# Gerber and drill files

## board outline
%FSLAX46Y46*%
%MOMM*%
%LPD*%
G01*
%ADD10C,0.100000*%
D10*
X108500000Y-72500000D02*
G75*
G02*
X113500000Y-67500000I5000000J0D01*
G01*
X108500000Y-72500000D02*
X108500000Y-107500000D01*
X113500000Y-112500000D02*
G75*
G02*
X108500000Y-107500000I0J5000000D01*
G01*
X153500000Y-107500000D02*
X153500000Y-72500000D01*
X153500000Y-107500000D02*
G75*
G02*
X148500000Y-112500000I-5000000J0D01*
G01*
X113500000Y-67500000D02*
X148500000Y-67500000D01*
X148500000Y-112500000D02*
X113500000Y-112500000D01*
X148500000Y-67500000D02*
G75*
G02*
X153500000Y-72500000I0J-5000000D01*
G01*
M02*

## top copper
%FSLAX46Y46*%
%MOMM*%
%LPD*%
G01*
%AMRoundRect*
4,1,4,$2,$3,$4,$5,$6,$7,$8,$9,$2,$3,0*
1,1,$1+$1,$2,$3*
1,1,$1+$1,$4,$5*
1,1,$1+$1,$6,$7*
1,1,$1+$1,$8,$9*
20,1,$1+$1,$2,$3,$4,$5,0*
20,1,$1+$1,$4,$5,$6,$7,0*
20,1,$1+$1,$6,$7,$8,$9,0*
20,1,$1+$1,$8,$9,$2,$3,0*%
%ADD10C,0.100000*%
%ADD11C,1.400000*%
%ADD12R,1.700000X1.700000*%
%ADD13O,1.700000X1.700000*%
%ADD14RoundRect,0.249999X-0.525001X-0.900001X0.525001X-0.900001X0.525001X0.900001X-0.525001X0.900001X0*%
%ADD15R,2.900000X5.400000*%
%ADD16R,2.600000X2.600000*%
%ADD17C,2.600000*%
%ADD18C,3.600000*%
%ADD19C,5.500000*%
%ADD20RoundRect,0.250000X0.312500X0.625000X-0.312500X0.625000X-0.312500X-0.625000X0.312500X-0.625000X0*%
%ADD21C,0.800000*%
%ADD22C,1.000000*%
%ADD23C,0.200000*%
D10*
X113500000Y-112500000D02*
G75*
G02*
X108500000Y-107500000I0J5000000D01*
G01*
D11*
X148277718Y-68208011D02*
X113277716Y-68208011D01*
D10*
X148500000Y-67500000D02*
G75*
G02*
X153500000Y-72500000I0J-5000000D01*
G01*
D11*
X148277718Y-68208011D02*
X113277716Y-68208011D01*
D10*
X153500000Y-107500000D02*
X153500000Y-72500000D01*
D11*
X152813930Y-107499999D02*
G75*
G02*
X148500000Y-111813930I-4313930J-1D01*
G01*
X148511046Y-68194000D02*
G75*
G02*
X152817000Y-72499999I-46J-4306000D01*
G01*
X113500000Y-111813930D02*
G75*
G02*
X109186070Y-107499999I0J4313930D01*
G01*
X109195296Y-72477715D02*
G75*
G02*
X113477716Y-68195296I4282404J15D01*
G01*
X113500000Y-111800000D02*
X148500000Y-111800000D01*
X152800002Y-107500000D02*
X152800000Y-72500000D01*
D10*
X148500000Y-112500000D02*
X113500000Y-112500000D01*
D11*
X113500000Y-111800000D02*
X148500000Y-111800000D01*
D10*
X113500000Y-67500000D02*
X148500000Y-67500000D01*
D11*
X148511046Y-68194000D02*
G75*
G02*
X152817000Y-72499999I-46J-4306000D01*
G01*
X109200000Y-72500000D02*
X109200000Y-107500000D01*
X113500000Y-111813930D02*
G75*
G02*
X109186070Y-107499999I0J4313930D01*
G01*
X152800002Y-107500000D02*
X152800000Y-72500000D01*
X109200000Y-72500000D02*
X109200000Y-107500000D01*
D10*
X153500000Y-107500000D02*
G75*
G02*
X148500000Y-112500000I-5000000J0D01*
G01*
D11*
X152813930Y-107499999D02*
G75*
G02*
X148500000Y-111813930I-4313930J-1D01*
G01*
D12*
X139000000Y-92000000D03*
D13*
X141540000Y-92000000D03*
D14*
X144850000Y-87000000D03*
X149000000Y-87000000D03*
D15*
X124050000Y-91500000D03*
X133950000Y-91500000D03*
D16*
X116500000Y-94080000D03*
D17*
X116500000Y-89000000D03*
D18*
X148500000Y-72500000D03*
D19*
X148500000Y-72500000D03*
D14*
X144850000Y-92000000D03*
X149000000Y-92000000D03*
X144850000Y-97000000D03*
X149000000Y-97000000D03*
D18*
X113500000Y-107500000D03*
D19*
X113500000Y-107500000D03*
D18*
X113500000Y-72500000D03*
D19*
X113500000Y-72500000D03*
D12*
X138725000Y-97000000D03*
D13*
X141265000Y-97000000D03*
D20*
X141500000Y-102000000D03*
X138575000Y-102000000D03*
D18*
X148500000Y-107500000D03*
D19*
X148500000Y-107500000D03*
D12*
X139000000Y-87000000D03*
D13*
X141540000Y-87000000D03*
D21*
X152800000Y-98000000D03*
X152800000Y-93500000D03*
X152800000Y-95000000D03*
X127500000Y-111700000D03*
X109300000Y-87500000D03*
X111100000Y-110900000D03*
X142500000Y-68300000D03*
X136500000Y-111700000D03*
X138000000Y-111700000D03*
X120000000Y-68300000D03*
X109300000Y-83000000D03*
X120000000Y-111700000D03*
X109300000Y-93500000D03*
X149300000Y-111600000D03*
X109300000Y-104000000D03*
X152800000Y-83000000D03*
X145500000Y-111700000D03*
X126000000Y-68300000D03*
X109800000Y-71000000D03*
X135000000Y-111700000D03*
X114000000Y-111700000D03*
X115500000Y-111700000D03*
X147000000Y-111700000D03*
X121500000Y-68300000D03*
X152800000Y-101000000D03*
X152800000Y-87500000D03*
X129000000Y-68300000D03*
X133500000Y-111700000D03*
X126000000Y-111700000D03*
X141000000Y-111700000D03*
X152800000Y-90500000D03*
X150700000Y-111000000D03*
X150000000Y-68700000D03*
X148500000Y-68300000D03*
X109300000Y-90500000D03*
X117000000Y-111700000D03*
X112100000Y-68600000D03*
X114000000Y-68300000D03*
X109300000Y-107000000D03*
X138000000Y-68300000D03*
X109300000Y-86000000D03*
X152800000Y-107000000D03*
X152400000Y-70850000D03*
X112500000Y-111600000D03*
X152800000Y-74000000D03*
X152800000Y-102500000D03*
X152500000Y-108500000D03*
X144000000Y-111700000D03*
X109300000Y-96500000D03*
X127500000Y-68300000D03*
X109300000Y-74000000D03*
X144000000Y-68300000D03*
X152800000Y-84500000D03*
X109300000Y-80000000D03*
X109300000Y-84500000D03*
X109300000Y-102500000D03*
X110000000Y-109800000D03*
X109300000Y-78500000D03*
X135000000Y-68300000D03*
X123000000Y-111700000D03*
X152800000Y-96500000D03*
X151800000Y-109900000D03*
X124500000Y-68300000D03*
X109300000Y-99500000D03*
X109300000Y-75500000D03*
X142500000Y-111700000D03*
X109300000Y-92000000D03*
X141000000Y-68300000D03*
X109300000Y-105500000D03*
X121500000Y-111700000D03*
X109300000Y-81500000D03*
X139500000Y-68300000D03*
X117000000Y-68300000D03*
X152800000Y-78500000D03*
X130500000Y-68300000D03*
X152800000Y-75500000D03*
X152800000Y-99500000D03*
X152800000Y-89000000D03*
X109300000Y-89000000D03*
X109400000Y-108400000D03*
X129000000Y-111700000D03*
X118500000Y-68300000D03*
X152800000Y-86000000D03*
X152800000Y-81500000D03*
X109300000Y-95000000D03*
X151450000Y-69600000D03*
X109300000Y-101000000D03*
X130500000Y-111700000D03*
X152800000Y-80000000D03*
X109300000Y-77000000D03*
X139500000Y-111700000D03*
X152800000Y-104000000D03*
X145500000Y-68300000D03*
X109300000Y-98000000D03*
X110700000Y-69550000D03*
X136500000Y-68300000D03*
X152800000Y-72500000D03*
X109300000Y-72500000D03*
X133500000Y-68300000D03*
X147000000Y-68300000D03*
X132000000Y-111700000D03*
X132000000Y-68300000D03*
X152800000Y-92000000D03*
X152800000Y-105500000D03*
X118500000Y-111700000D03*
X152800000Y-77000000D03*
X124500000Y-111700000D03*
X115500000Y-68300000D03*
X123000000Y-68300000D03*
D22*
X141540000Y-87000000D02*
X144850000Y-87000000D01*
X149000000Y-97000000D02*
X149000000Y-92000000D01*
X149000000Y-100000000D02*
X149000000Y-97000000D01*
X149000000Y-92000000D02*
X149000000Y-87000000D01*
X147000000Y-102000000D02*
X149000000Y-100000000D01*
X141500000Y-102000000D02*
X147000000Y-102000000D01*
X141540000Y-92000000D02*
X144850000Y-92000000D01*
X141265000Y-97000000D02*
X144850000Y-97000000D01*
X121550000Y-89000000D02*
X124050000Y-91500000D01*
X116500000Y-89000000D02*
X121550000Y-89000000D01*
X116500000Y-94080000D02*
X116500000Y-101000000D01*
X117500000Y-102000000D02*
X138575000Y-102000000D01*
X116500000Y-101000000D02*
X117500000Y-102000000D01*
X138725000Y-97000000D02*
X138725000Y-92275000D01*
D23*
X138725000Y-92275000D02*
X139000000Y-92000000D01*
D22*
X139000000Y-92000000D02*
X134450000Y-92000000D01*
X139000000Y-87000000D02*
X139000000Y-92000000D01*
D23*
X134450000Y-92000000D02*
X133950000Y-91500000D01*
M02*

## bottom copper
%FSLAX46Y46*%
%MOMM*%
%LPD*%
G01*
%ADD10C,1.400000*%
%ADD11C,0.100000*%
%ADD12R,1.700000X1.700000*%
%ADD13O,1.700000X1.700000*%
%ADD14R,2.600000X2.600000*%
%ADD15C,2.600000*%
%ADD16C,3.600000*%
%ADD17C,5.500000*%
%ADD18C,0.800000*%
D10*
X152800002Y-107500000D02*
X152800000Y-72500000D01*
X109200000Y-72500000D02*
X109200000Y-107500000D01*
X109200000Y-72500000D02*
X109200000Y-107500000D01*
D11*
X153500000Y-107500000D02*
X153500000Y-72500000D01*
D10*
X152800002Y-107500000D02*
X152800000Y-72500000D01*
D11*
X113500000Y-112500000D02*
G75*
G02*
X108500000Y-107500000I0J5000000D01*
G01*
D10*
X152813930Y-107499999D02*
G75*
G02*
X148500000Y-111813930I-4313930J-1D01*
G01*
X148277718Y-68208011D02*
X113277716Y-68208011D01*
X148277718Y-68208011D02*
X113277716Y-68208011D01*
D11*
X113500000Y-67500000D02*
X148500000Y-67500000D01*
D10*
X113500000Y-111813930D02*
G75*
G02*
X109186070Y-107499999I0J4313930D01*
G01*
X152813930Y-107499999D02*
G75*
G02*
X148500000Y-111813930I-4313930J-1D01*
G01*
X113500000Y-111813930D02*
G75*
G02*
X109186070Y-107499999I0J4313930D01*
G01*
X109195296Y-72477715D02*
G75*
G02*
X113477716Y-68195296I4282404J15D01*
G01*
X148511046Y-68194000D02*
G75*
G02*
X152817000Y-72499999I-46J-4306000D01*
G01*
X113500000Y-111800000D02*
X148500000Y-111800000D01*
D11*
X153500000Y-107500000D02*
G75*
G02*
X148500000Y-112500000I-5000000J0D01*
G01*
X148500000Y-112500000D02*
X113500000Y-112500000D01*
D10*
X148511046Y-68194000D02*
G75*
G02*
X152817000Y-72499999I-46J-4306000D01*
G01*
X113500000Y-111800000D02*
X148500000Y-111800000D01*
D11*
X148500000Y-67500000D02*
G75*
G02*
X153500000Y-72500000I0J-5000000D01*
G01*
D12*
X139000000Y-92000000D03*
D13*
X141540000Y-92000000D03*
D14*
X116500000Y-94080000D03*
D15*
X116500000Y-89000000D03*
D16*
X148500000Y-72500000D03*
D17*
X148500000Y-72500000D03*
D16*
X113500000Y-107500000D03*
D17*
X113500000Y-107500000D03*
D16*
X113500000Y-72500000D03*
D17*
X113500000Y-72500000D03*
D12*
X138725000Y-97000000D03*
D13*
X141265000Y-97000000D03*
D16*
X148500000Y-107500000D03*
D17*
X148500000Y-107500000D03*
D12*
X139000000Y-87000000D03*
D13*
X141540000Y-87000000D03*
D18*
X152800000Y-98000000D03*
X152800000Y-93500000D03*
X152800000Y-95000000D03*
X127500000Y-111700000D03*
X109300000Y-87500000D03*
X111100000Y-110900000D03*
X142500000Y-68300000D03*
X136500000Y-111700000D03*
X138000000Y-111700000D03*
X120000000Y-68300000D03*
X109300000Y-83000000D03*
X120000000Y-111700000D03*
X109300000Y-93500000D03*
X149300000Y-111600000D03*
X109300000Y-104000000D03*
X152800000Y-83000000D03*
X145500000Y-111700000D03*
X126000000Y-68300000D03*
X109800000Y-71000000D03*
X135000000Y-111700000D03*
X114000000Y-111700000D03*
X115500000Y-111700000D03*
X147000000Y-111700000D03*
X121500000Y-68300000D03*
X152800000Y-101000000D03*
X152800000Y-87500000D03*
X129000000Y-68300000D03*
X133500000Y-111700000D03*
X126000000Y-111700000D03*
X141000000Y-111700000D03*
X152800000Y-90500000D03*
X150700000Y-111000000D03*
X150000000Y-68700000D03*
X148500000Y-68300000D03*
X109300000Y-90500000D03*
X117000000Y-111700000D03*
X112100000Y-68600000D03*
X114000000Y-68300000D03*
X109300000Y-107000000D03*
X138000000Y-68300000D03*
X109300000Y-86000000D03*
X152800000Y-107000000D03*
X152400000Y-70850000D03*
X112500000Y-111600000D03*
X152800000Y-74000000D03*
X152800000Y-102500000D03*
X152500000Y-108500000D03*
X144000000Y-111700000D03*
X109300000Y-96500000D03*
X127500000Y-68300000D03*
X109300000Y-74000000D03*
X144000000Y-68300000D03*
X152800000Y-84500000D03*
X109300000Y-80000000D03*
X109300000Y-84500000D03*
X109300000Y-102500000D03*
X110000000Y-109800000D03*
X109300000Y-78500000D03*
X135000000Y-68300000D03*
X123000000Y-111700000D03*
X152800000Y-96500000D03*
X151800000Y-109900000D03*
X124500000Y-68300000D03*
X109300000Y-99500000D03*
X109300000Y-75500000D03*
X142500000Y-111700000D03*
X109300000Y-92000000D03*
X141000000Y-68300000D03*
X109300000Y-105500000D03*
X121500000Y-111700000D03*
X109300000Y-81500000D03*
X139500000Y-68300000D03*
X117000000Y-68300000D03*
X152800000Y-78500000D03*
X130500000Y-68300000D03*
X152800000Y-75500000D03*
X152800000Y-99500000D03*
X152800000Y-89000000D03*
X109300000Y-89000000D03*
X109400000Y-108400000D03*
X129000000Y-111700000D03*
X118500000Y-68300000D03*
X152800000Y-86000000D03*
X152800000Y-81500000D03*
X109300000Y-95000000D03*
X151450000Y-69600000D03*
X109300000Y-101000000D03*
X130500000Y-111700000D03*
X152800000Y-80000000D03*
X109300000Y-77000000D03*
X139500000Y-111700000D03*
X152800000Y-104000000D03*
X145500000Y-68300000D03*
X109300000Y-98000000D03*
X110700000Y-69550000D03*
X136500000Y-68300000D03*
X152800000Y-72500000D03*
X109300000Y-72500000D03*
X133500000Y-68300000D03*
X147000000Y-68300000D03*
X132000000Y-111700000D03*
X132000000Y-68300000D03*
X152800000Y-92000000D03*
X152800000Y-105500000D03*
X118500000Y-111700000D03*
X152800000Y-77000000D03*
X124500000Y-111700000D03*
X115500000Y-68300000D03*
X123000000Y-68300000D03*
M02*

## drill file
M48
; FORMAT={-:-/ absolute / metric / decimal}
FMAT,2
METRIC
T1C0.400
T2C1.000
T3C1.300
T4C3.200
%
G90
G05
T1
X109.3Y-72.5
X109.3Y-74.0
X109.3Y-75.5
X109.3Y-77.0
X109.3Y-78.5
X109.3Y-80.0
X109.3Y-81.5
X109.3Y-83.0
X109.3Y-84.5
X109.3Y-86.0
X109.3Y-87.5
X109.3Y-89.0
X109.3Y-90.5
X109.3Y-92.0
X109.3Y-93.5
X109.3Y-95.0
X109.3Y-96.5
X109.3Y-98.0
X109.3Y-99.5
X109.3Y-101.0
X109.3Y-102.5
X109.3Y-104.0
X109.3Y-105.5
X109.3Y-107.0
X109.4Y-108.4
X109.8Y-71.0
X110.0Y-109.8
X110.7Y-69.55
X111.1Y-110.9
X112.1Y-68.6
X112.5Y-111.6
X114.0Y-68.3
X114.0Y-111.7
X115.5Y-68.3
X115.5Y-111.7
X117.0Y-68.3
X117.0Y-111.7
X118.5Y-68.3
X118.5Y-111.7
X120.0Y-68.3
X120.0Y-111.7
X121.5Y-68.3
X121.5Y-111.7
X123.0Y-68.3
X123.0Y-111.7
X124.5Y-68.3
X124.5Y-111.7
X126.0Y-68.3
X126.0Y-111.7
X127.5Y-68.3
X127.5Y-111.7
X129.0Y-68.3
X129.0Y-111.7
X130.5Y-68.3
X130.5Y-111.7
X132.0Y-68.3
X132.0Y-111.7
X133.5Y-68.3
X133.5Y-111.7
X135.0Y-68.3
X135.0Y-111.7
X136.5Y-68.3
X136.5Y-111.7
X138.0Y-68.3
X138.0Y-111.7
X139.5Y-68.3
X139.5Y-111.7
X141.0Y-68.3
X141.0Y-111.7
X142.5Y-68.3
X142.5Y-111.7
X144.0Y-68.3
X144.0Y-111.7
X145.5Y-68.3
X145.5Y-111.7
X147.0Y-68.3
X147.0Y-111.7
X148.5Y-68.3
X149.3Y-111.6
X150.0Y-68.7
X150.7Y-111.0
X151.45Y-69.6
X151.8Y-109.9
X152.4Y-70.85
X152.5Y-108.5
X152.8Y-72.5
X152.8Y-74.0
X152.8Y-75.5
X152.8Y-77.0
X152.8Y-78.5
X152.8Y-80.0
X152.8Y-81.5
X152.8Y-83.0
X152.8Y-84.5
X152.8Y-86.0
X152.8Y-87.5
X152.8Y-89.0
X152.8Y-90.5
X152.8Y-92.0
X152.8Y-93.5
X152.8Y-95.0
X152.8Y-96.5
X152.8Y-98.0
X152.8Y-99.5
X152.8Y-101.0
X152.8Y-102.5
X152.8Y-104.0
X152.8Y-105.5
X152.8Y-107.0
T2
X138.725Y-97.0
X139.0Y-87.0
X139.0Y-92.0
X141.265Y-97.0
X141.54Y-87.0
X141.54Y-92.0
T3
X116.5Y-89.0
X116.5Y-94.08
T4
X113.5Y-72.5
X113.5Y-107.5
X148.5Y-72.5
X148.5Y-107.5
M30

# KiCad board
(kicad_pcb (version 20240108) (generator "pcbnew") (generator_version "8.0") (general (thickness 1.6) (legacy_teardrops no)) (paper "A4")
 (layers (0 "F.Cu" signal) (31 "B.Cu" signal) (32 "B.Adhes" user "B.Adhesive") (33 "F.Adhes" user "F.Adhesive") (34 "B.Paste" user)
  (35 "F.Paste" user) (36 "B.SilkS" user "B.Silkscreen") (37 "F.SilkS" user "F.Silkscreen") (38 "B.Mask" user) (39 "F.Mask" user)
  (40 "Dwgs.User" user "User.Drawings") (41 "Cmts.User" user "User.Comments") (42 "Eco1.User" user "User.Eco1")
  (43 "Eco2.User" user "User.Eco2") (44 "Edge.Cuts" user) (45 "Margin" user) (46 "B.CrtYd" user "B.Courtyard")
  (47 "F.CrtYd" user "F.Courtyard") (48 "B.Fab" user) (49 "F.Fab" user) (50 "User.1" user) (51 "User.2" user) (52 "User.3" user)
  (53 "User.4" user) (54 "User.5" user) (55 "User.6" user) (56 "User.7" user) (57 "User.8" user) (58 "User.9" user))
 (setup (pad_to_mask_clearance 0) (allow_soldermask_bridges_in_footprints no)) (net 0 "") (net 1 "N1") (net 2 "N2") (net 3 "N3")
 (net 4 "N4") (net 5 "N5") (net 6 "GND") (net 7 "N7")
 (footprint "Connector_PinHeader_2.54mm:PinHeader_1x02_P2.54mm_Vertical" (layer "F.Cu") (at 139 92 90)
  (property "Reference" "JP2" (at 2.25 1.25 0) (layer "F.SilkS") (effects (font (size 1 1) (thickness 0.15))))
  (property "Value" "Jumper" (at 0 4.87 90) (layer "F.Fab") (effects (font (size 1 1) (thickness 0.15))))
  (pad "1" thru_hole rect (at 0 0 90) (size 1.7 1.7) (drill 1) (layers "*.Cu" "*.Mask") (remove_unused_layers no) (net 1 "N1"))
  (pad "2" thru_hole oval (at 0 2.54 90) (size 1.7 1.7) (drill 1) (layers "*.Cu" "*.Mask") (remove_unused_layers no) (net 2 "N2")))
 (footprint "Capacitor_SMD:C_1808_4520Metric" (layer "F.Cu") (at 146.925 87)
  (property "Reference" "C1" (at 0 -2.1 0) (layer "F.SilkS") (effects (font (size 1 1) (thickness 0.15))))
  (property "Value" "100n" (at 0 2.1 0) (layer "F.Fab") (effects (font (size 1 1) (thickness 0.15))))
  (pad "1" smd roundrect (at -2.075 0) (size 1.55 2.3) (layers "F.Cu" "F.Paste" "F.Mask") (roundrect_rratio 0.16129) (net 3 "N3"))
  (pad "2" smd roundrect (at 2.075 0) (size 1.55 2.3) (layers "F.Cu" "F.Paste" "F.Mask") (roundrect_rratio 0.16129) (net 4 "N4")))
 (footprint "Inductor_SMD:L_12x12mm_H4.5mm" (layer "F.Cu") (at 129 91.5)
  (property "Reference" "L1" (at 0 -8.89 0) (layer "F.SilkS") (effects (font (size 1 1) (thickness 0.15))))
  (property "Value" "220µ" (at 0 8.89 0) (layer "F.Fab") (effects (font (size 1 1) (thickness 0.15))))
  (pad "1" smd rect (at -4.95 0) (size 2.9 5.4) (layers "F.Cu" "F.Paste" "F.Mask") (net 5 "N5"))
  (pad "2" smd rect (at 4.95 0) (size 2.9 5.4) (layers "F.Cu" "F.Paste" "F.Mask") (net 1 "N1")))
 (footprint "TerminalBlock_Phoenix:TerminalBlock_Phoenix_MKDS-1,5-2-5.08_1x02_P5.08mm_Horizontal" (layer "F.Cu") (at 116.5 94.08 90)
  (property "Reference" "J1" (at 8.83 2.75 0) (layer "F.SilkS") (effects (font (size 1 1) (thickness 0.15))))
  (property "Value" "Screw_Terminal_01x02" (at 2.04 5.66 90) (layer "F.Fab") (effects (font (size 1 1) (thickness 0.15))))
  (pad "1" thru_hole rect (at 0 0 90) (size 2.6 2.6) (drill 1.3) (layers "*.Cu" "*.Mask") (remove_unused_layers no) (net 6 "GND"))
  (pad "2" thru_hole circle (at 5.08 0 90) (size 2.6 2.6) (drill 1.3) (layers "*.Cu" "*.Mask") (remove_unused_layers no) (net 5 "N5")))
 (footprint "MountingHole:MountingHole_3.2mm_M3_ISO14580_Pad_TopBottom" (layer "F.Cu") (at 148.5 72.5)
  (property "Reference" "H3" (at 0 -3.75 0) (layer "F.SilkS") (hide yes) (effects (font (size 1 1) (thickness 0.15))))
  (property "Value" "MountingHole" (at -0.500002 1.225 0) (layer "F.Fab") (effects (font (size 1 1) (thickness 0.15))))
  (pad "1" thru_hole circle (at 0 0) (size 3.6 3.6) (drill 3.2) (layers "*.Cu" "*.Mask") (remove_unused_layers no))
  (pad "1" connect circle (at 0 0) (size 5.5 5.5) (layers "F.Cu" "F.Mask"))
  (pad "1" connect circle (at 0 0) (size 5.5 5.5) (layers "B.Cu" "B.Mask")))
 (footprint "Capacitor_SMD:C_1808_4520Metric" (layer "F.Cu") (at 146.925 92)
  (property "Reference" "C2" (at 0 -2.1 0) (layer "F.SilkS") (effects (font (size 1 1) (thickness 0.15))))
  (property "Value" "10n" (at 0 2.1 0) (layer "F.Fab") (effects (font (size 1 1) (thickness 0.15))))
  (pad "1" smd roundrect (at -2.075 0) (size 1.55 2.3) (layers "F.Cu" "F.Paste" "F.Mask") (roundrect_rratio 0.16129) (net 2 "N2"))
  (pad "2" smd roundrect (at 2.075 0) (size 1.55 2.3) (layers "F.Cu" "F.Paste" "F.Mask") (roundrect_rratio 0.16129) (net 4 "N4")))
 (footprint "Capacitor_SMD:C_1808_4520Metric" (layer "F.Cu") (at 146.925 97)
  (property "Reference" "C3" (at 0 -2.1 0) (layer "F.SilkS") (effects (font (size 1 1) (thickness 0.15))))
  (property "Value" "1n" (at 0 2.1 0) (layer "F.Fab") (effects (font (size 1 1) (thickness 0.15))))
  (pad "1" smd roundrect (at -2.075 0) (size 1.55 2.3) (layers "F.Cu" "F.Paste" "F.Mask") (roundrect_rratio 0.16129) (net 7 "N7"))
  (pad "2" smd roundrect (at 2.075 0) (size 1.55 2.3) (layers "F.Cu" "F.Paste" "F.Mask") (roundrect_rratio 0.16129) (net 4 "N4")))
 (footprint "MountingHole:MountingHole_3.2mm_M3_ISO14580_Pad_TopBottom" (layer "F.Cu") (at 113.5 107.5 -90)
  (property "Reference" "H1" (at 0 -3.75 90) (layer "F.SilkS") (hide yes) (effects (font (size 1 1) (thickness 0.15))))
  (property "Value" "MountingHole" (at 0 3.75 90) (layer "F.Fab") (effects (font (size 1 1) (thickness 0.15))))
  (pad "1" thru_hole circle (at 0 0 270) (size 3.6 3.6) (drill 3.2) (layers "*.Cu" "*.Mask") (remove_unused_layers no))
  (pad "1" connect circle (at 0 0 270) (size 5.5 5.5) (layers "F.Cu" "F.Mask"))
  (pad "1" connect circle (at 0 0 270) (size 5.5 5.5) (layers "B.Cu" "B.Mask")))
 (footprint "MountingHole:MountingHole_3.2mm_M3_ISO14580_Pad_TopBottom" (layer "F.Cu") (at 113.5 72.5)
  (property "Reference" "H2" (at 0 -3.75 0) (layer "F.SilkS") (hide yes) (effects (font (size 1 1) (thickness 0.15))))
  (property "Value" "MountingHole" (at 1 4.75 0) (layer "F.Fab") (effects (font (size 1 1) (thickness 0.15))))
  (pad "1" thru_hole circle (at 0 0) (size 3.6 3.6) (drill 3.2) (layers "*.Cu" "*.Mask") (remove_unused_layers no))
  (pad "1" connect circle (at 0 0) (size 5.5 5.5) (layers "F.Cu" "F.Mask"))
  (pad "1" connect circle (at 0 0) (size 5.5 5.5) (layers "B.Cu" "B.Mask")))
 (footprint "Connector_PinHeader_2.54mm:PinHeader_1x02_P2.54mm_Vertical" (layer "F.Cu") (at 138.725 97 90)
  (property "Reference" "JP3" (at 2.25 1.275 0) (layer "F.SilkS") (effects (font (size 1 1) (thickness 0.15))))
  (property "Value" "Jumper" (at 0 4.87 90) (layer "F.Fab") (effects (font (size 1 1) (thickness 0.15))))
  (pad "1" thru_hole rect (at 0 0 90) (size 1.7 1.7) (drill 1) (layers "*.Cu" "*.Mask") (remove_unused_layers no) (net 1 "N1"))
  (pad "2" thru_hole oval (at 0 2.54 90) (size 1.7 1.7) (drill 1) (layers "*.Cu" "*.Mask") (remove_unused_layers no) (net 7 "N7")))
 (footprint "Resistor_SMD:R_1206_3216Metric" (layer "F.Cu") (at 140.0375 102 180)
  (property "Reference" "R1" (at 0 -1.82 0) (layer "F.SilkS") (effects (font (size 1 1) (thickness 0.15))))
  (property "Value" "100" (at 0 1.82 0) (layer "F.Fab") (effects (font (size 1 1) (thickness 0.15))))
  (pad "1" smd roundrect (at -1.4625 0 180) (size 1.125 1.75) (layers "F.Cu" "F.Paste" "F.Mask") (roundrect_rratio 0.222222) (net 4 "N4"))
  (pad "2" smd roundrect (at 1.4625 0 180) (size 1.125 1.75) (layers "F.Cu" "F.Paste" "F.Mask") (roundrect_rratio 0.222222) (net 6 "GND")))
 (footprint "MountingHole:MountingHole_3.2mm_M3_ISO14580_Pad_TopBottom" (layer "F.Cu") (at 148.5 107.5)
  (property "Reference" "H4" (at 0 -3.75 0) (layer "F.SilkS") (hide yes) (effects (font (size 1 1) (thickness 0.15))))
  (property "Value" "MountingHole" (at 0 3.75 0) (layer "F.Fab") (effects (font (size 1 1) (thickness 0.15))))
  (pad "1" thru_hole circle (at 0 0) (size 3.6 3.6) (drill 3.2) (layers "*.Cu" "*.Mask") (remove_unused_layers no))
  (pad "1" connect circle (at 0 0) (size 5.5 5.5) (layers "F.Cu" "F.Mask"))
  (pad "1" connect circle (at 0 0) (size 5.5 5.5) (layers "B.Cu" "B.Mask")))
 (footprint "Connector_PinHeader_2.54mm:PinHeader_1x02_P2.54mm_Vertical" (layer "F.Cu") (at 139 87 90)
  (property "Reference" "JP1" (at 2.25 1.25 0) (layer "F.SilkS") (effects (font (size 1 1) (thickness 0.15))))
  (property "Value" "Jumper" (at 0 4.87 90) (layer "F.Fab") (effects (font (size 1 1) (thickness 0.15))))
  (pad "1" thru_hole rect (at 0 0 90) (size 1.7 1.7) (drill 1) (layers "*.Cu" "*.Mask") (remove_unused_layers no) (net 1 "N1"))
  (pad "2" thru_hole oval (at 0 2.54 90) (size 1.7 1.7) (drill 1) (layers "*.Cu" "*.Mask") (remove_unused_layers no) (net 3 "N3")))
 (gr_arc (start 113.5 112.5) (mid 109.964466 111.035534) (end 108.5 107.5) (stroke (width 0.1) (type default)) (layer "F.Cu") (net 6))
 (gr_line (start 148.277718 68.208011) (end 113.277716 68.208011) (stroke (width 1.4) (type default)) (layer "F.Cu") (net 6))
 (gr_arc (start 148.5 67.5) (mid 152.035517 68.964473) (end 153.5 72.5) (stroke (width 0.1) (type default)) (layer "F.Cu") (net 6))
 (gr_line (start 148.277718 68.208011) (end 113.277716 68.208011) (stroke (width 1.4) (type default)) (layer "F.Cu") (net 6))
 (gr_line (start 153.5 107.5) (end 153.5 72.5) (stroke (width 0.1) (type default)) (layer "F.Cu") (net 6))
 (gr_arc (start 152.81393 107.499999) (mid 151.55041 110.55041) (end 148.5 111.81393) (stroke (width 1.4) (type default)) (layer "F.Cu")
  (net 6))
 (gr_arc (start 148.511046 68.194) (mid 151.555847 69.455199) (end 152.817046 72.499999) (stroke (width 1.4) (type default)) (layer "F.Cu")
  (net 6))
 (gr_arc (start 113.5 111.81393) (mid 110.44959 110.550409) (end 109.18607 107.499999) (stroke (width 1.4) (type default)) (layer "F.Cu")
  (net 6))
 (gr_arc (start 109.195296 72.477715) (mid 110.449583 69.449583) (end 113.477716 68.195296) (stroke (width 1.4) (type default))
  (layer "F.Cu") (net 6))
 (gr_line (start 113.5 111.8) (end 148.5 111.8) (stroke (width 1.4) (type default)) (layer "F.Cu") (net 6))
 (gr_line (start 152.800002 107.5) (end 152.8 72.5) (stroke (width 1.4) (type default)) (layer "F.Cu") (net 6))
 (gr_line (start 148.5 112.5) (end 113.5 112.5) (stroke (width 0.1) (type default)) (layer "F.Cu") (net 6))
 (gr_line (start 113.5 111.8) (end 148.5 111.8) (stroke (width 1.4) (type default)) (layer "F.Cu") (net 6))
 (gr_line (start 113.5 67.5) (end 148.5 67.5) (stroke (width 0.1) (type default)) (layer "F.Cu") (net 6))
 (gr_arc (start 148.511046 68.194) (mid 151.555836 69.455215) (end 152.817046 72.499999) (stroke (width 1.4) (type default)) (layer "F.Cu")
  (net 6))
 (gr_line (start 109.2 72.5) (end 109.2 107.5) (stroke (width 1.4) (type default)) (layer "F.Cu") (net 6))
 (gr_arc (start 113.5 111.81393) (mid 110.44959 110.550409) (end 109.18607 107.499999) (stroke (width 1.4) (type default)) (layer "F.Cu")
  (net 6))
 (gr_line (start 152.800002 107.5) (end 152.8 72.5) (stroke (width 1.4) (type default)) (layer "F.Cu") (net 6))
 (gr_line (start 109.2 72.5) (end 109.2 107.5) (stroke (width 1.4) (type default)) (layer "F.Cu") (net 6))
 (gr_arc (start 153.5 107.5) (mid 152.035535 111.035535) (end 148.5 112.5) (stroke (width 0.1) (type default)) (layer "F.Cu") (net 6))
 (gr_arc (start 152.81393 107.499999) (mid 151.55041 110.55041) (end 148.5 111.81393) (stroke (width 1.4) (type default)) (layer "F.Cu")
  (net 6))
 (gr_line (start 152.800002 107.5) (end 152.8 72.5) (stroke (width 1.4) (type default)) (layer "B.Cu") (net 6))
 (gr_line (start 109.2 72.5) (end 109.2 107.5) (stroke (width 1.4) (type default)) (layer "B.Cu") (net 6))
 (gr_line (start 109.2 72.5) (end 109.2 107.5) (stroke (width 1.4) (type default)) (layer "B.Cu") (net 6))
 (gr_line (start 153.5 107.5) (end 153.5 72.5) (stroke (width 0.1) (type default)) (layer "B.Cu") (net 6))
 (gr_line (start 152.800002 107.5) (end 152.8 72.5) (stroke (width 1.4) (type default)) (layer "B.Cu") (net 6))
 (gr_arc (start 113.5 112.5) (mid 109.964466 111.035534) (end 108.5 107.5) (stroke (width 0.1) (type default)) (layer "B.Cu") (net 6))
 (gr_arc (start 152.81393 107.499999) (mid 151.55041 110.55041) (end 148.5 111.81393) (stroke (width 1.4) (type default)) (layer "B.Cu")
  (net 6))
 (gr_line (start 148.277718 68.208011) (end 113.277716 68.208011) (stroke (width 1.4) (type default)) (layer "B.Cu") (net 6))
 (gr_line (start 148.277718 68.208011) (end 113.277716 68.208011) (stroke (width 1.4) (type default)) (layer "B.Cu") (net 6))
 (gr_line (start 113.5 67.5) (end 148.5 67.5) (stroke (width 0.1) (type default)) (layer "B.Cu") (net 6))
 (gr_arc (start 113.5 111.81393) (mid 110.44959 110.550409) (end 109.18607 107.499999) (stroke (width 1.4) (type default)) (layer "B.Cu")
  (net 6))
 (gr_arc (start 152.81393 107.499999) (mid 151.55041 110.55041) (end 148.5 111.81393) (stroke (width 1.4) (type default)) (layer "B.Cu")
  (net 6))
 (gr_arc (start 113.5 111.81393) (mid 110.44959 110.550409) (end 109.18607 107.499999) (stroke (width 1.4) (type default)) (layer "B.Cu")
  (net 6))
 (gr_arc (start 109.195296 72.477715) (mid 110.449583 69.449583) (end 113.477716 68.195296) (stroke (width 1.4) (type default))
  (layer "B.Cu") (net 6))
 (gr_arc (start 148.511046 68.194) (mid 151.555847 69.455199) (end 152.817046 72.499999) (stroke (width 1.4) (type default)) (layer "B.Cu")
  (net 6))
 (gr_line (start 113.5 111.8) (end 148.5 111.8) (stroke (width 1.4) (type default)) (layer "B.Cu") (net 6))
 (gr_arc (start 153.5 107.5) (mid 152.035535 111.035535) (end 148.5 112.5) (stroke (width 0.1) (type default)) (layer "B.Cu") (net 6))
 (gr_line (start 148.5 112.5) (end 113.5 112.5) (stroke (width 0.1) (type default)) (layer "B.Cu") (net 6))
 (gr_arc (start 148.511046 68.194) (mid 151.555836 69.455215) (end 152.817046 72.499999) (stroke (width 1.4) (type default)) (layer "B.Cu")
  (net 6))
 (gr_line (start 113.5 111.8) (end 148.5 111.8) (stroke (width 1.4) (type default)) (layer "B.Cu") (net 6))
 (gr_arc (start 148.5 67.5) (mid 152.035517 68.964473) (end 153.5 72.5) (stroke (width 0.1) (type default)) (layer "B.Cu") (net 6))
 (gr_arc (start 108.5 72.5) (mid 109.964466 68.964466) (end 113.5 67.5) (stroke (width 0.1) (type default)) (layer "Edge.Cuts"))
 (gr_line (start 108.5 72.5) (end 108.5 107.5) (stroke (width 0.1) (type default)) (layer "Edge.Cuts"))
 (gr_arc (start 113.5 112.5) (mid 109.964466 111.035534) (end 108.5 107.5) (stroke (width 0.1) (type default)) (layer "Edge.Cuts"))
 (gr_line (start 153.5 107.5) (end 153.5 72.5) (stroke (width 0.1) (type default)) (layer "Edge.Cuts"))
 (gr_arc (start 153.5 107.5) (mid 152.035534 111.035534) (end 148.5 112.5) (stroke (width 0.1) (type default)) (layer "Edge.Cuts"))
 (gr_line (start 113.5 67.5) (end 148.5 67.5) (stroke (width 0.1) (type default)) (layer "Edge.Cuts"))
 (gr_line (start 148.5 112.5) (end 113.5 112.5) (stroke (width 0.1) (type default)) (layer "Edge.Cuts"))
 (gr_arc (start 148.5 67.5) (mid 152.035534 68.964466) (end 153.5 72.5) (stroke (width 0.1) (type default)) (layer "Edge.Cuts"))
 (segment (start 141.54 87) (end 144.85 87) (width 1) (layer "F.Cu") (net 3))
 (segment (start 149 97) (end 149 92) (width 1) (layer "F.Cu") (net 4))
 (segment (start 149 100) (end 149 97) (width 1) (layer "F.Cu") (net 4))
 (segment (start 149 92) (end 149 87) (width 1) (layer "F.Cu") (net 4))
 (segment (start 147 102) (end 149 100) (width 1) (layer "F.Cu") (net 4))
 (segment (start 141.5 102) (end 147 102) (width 1) (layer "F.Cu") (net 4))
 (segment (start 141.54 92) (end 144.85 92) (width 1) (layer "F.Cu") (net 2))
 (segment (start 141.265 97) (end 144.85 97) (width 1) (layer "F.Cu") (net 7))
 (segment (start 121.55 89) (end 124.05 91.5) (width 1) (layer "F.Cu") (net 5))
 (segment (start 116.5 89) (end 121.55 89) (width 1) (layer "F.Cu") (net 5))
 (segment (start 116.5 94.08) (end 116.5 101) (width 1) (layer "F.Cu") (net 6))
 (segment (start 117.5 102) (end 138.575 102) (width 1) (layer "F.Cu") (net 6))
 (segment (start 116.5 101) (end 117.5 102) (width 1) (layer "F.Cu") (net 6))
 (via (at 152.8 98) (size 0.8) (drill 0.4) (layers "F.Cu" "B.Cu") (free yes) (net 6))
 (via (at 152.8 93.5) (size 0.8) (drill 0.4) (layers "F.Cu" "B.Cu") (free yes) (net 6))
 (via (at 152.8 95) (size 0.8) (drill 0.4) (layers "F.Cu" "B.Cu") (free yes) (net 6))
 (via (at 127.5 111.7) (size 0.8) (drill 0.4) (layers "F.Cu" "B.Cu") (free yes) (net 6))
 (via (at 109.3 87.5) (size 0.8) (drill 0.4) (layers "F.Cu" "B.Cu") (free yes) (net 6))
 (via (at 111.1 110.9) (size 0.8) (drill 0.4) (layers "F.Cu" "B.Cu") (free yes) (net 6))
 (via (at 142.5 68.3) (size 0.8) (drill 0.4) (layers "F.Cu" "B.Cu") (free yes) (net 6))
 (via (at 136.5 111.7) (size 0.8) (drill 0.4) (layers "F.Cu" "B.Cu") (free yes) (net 6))
 (via (at 138 111.7) (size 0.8) (drill 0.4) (layers "F.Cu" "B.Cu") (free yes) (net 6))
 (via (at 120 68.3) (size 0.8) (drill 0.4) (layers "F.Cu" "B.Cu") (free yes) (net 6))
 (via (at 109.3 83) (size 0.8) (drill 0.4) (layers "F.Cu" "B.Cu") (free yes) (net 6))
 (via (at 120 111.7) (size 0.8) (drill 0.4) (layers "F.Cu" "B.Cu") (free yes) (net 6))
 (via (at 109.3 93.5) (size 0.8) (drill 0.4) (layers "F.Cu" "B.Cu") (free yes) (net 6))
 (via (at 149.3 111.6) (size 0.8) (drill 0.4) (layers "F.Cu" "B.Cu") (free yes) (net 6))
 (via (at 109.3 104) (size 0.8) (drill 0.4) (layers "F.Cu" "B.Cu") (free yes) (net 6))
 (via (at 152.8 83) (size 0.8) (drill 0.4) (layers "F.Cu" "B.Cu") (free yes) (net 6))
 (via (at 145.5 111.7) (size 0.8) (drill 0.4) (layers "F.Cu" "B.Cu") (free yes) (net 6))
 (via (at 126 68.3) (size 0.8) (drill 0.4) (layers "F.Cu" "B.Cu") (free yes) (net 6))
 (via (at 109.8 71) (size 0.8) (drill 0.4) (layers "F.Cu" "B.Cu") (free yes) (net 6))
 (via (at 135 111.7) (size 0.8) (drill 0.4) (layers "F.Cu" "B.Cu") (free yes) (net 6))
 (via (at 114 111.7) (size 0.8) (drill 0.4) (layers "F.Cu" "B.Cu") (free yes) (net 6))
 (via (at 115.5 111.7) (size 0.8) (drill 0.4) (layers "F.Cu" "B.Cu") (free yes) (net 6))
 (via (at 147 111.7) (size 0.8) (drill 0.4) (layers "F.Cu" "B.Cu") (free yes) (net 6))
 (via (at 121.5 68.3) (size 0.8) (drill 0.4) (layers "F.Cu" "B.Cu") (free yes) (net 6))
 (via (at 152.8 101) (size 0.8) (drill 0.4) (layers "F.Cu" "B.Cu") (free yes) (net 6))
 (via (at 152.8 87.5) (size 0.8) (drill 0.4) (layers "F.Cu" "B.Cu") (free yes) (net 6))
 (via (at 129 68.3) (size 0.8) (drill 0.4) (layers "F.Cu" "B.Cu") (free yes) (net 6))
 (via (at 133.5 111.7) (size 0.8) (drill 0.4) (layers "F.Cu" "B.Cu") (free yes) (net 6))
 (via (at 126 111.7) (size 0.8) (drill 0.4) (layers "F.Cu" "B.Cu") (free yes) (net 6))
 (via (at 141 111.7) (size 0.8) (drill 0.4) (layers "F.Cu" "B.Cu") (free yes) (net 6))
 (via (at 152.8 90.5) (size 0.8) (drill 0.4) (layers "F.Cu" "B.Cu") (free yes) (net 6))
 (via (at 150.7 111) (size 0.8) (drill 0.4) (layers "F.Cu" "B.Cu") (free yes) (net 6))
 (via (at 150 68.7) (size 0.8) (drill 0.4) (layers "F.Cu" "B.Cu") (free yes) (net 6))
 (via (at 148.5 68.3) (size 0.8) (drill 0.4) (layers "F.Cu" "B.Cu") (free yes) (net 6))
 (via (at 109.3 90.5) (size 0.8) (drill 0.4) (layers "F.Cu" "B.Cu") (free yes) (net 6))
 (via (at 117 111.7) (size 0.8) (drill 0.4) (layers "F.Cu" "B.Cu") (free yes) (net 6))
 (via (at 112.1 68.6) (size 0.8) (drill 0.4) (layers "F.Cu" "B.Cu") (free yes) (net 6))
 (via (at 114 68.3) (size 0.8) (drill 0.4) (layers "F.Cu" "B.Cu") (free yes) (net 6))
 (via (at 109.3 107) (size 0.8) (drill 0.4) (layers "F.Cu" "B.Cu") (free yes) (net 6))
 (via (at 138 68.3) (size 0.8) (drill 0.4) (layers "F.Cu" "B.Cu") (free yes) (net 6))
 (via (at 109.3 86) (size 0.8) (drill 0.4) (layers "F.Cu" "B.Cu") (free yes) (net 6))
 (via (at 152.8 107) (size 0.8) (drill 0.4) (layers "F.Cu" "B.Cu") (free yes) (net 6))
 (via (at 152.4 70.85) (size 0.8) (drill 0.4) (layers "F.Cu" "B.Cu") (free yes) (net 6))
 (via (at 112.5 111.6) (size 0.8) (drill 0.4) (layers "F.Cu" "B.Cu") (free yes) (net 6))
 (via (at 152.8 74) (size 0.8) (drill 0.4) (layers "F.Cu" "B.Cu") (free yes) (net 6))
 (via (at 152.8 102.5) (size 0.8) (drill 0.4) (layers "F.Cu" "B.Cu") (free yes) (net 6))
 (via (at 152.5 108.5) (size 0.8) (drill 0.4) (layers "F.Cu" "B.Cu") (free yes) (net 6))
 (via (at 144 111.7) (size 0.8) (drill 0.4) (layers "F.Cu" "B.Cu") (free yes) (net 6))
 (via (at 109.3 96.5) (size 0.8) (drill 0.4) (layers "F.Cu" "B.Cu") (free yes) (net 6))
 (via (at 127.5 68.3) (size 0.8) (drill 0.4) (layers "F.Cu" "B.Cu") (free yes) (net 6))
 (via (at 109.3 74) (size 0.8) (drill 0.4) (layers "F.Cu" "B.Cu") (free yes) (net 6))
 (via (at 144 68.3) (size 0.8) (drill 0.4) (layers "F.Cu" "B.Cu") (free yes) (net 6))
 (via (at 152.8 84.5) (size 0.8) (drill 0.4) (layers "F.Cu" "B.Cu") (free yes) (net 6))
 (via (at 109.3 80) (size 0.8) (drill 0.4) (layers "F.Cu" "B.Cu") (free yes) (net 6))
 (via (at 109.3 84.5) (size 0.8) (drill 0.4) (layers "F.Cu" "B.Cu") (free yes) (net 6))
 (via (at 109.3 102.5) (size 0.8) (drill 0.4) (layers "F.Cu" "B.Cu") (free yes) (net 6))
 (via (at 110 109.8) (size 0.8) (drill 0.4) (layers "F.Cu" "B.Cu") (free yes) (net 6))
 (via (at 109.3 78.5) (size 0.8) (drill 0.4) (layers "F.Cu" "B.Cu") (free yes) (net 6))
 (via (at 135 68.3) (size 0.8) (drill 0.4) (layers "F.Cu" "B.Cu") (free yes) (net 6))
 (via (at 123 111.7) (size 0.8) (drill 0.4) (layers "F.Cu" "B.Cu") (free yes) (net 6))
 (via (at 152.8 96.5) (size 0.8) (drill 0.4) (layers "F.Cu" "B.Cu") (free yes) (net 6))
 (via (at 151.8 109.9) (size 0.8) (drill 0.4) (layers "F.Cu" "B.Cu") (free yes) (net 6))
 (via (at 124.5 68.3) (size 0.8) (drill 0.4) (layers "F.Cu" "B.Cu") (free yes) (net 6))
 (via (at 109.3 99.5) (size 0.8) (drill 0.4) (layers "F.Cu" "B.Cu") (free yes) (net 6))
 (via (at 109.3 75.5) (size 0.8) (drill 0.4) (layers "F.Cu" "B.Cu") (free yes) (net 6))
 (via (at 142.5 111.7) (size 0.8) (drill 0.4) (layers "F.Cu" "B.Cu") (free yes) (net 6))
 (via (at 109.3 92) (size 0.8) (drill 0.4) (layers "F.Cu" "B.Cu") (free yes) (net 6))
 (via (at 141 68.3) (size 0.8) (drill 0.4) (layers "F.Cu" "B.Cu") (free yes) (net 6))
 (via (at 109.3 105.5) (size 0.8) (drill 0.4) (layers "F.Cu" "B.Cu") (free yes) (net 6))
 (via (at 121.5 111.7) (size 0.8) (drill 0.4) (layers "F.Cu" "B.Cu") (free yes) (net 6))
 (via (at 109.3 81.5) (size 0.8) (drill 0.4) (layers "F.Cu" "B.Cu") (free yes) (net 6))
 (via (at 139.5 68.3) (size 0.8) (drill 0.4) (layers "F.Cu" "B.Cu") (free yes) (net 6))
 (via (at 117 68.3) (size 0.8) (drill 0.4) (layers "F.Cu" "B.Cu") (free yes) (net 6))
 (via (at 152.8 78.5) (size 0.8) (drill 0.4) (layers "F.Cu" "B.Cu") (free yes) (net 6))
 (via (at 130.5 68.3) (size 0.8) (drill 0.4) (layers "F.Cu" "B.Cu") (free yes) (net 6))
 (via (at 152.8 75.5) (size 0.8) (drill 0.4) (layers "F.Cu" "B.Cu") (free yes) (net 6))
 (via (at 152.8 99.5) (size 0.8) (drill 0.4) (layers "F.Cu" "B.Cu") (free yes) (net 6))
 (via (at 152.8 89) (size 0.8) (drill 0.4) (layers "F.Cu" "B.Cu") (free yes) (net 6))
 (via (at 109.3 89) (size 0.8) (drill 0.4) (layers "F.Cu" "B.Cu") (free yes) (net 6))
 (via (at 109.4 108.4) (size 0.8) (drill 0.4) (layers "F.Cu" "B.Cu") (free yes) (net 6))
 (via (at 129 111.7) (size 0.8) (drill 0.4) (layers "F.Cu" "B.Cu") (free yes) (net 6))
 (via (at 118.5 68.3) (size 0.8) (drill 0.4) (layers "F.Cu" "B.Cu") (free yes) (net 6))
 (via (at 152.8 86) (size 0.8) (drill 0.4) (layers "F.Cu" "B.Cu") (free yes) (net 6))
 (via (at 152.8 81.5) (size 0.8) (drill 0.4) (layers "F.Cu" "B.Cu") (free yes) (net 6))
 (via (at 109.3 95) (size 0.8) (drill 0.4) (layers "F.Cu" "B.Cu") (free yes) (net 6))
 (via (at 151.45 69.6) (size 0.8) (drill 0.4) (layers "F.Cu" "B.Cu") (free yes) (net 6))
 (via (at 109.3 101) (size 0.8) (drill 0.4) (layers "F.Cu" "B.Cu") (free yes) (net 6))
 (via (at 130.5 111.7) (size 0.8) (drill 0.4) (layers "F.Cu" "B.Cu") (free yes) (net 6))
 (via (at 152.8 80) (size 0.8) (drill 0.4) (layers "F.Cu" "B.Cu") (free yes) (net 6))
 (via (at 109.3 77) (size 0.8) (drill 0.4) (layers "F.Cu" "B.Cu") (free yes) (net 6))
 (via (at 139.5 111.7) (size 0.8) (drill 0.4) (layers "F.Cu" "B.Cu") (free yes) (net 6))
 (via (at 152.8 104) (size 0.8) (drill 0.4) (layers "F.Cu" "B.Cu") (free yes) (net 6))
 (via (at 145.5 68.3) (size 0.8) (drill 0.4) (layers "F.Cu" "B.Cu") (free yes) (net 6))
 (via (at 109.3 98) (size 0.8) (drill 0.4) (layers "F.Cu" "B.Cu") (free yes) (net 6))
 (via (at 110.7 69.55) (size 0.8) (drill 0.4) (layers "F.Cu" "B.Cu") (free yes) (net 6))
 (via (at 136.5 68.3) (size 0.8) (drill 0.4) (layers "F.Cu" "B.Cu") (free yes) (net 6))
 (via (at 152.8 72.5) (size 0.8) (drill 0.4) (layers "F.Cu" "B.Cu") (free yes) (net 6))
 (via (at 109.3 72.5) (size 0.8) (drill 0.4) (layers "F.Cu" "B.Cu") (free yes) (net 6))
 (via (at 133.5 68.3) (size 0.8) (drill 0.4) (layers "F.Cu" "B.Cu") (free yes) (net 6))
 (via (at 147 68.3) (size 0.8) (drill 0.4) (layers "F.Cu" "B.Cu") (free yes) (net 6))
 (via (at 132 111.7) (size 0.8) (drill 0.4) (layers "F.Cu" "B.Cu") (free yes) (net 6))
 (via (at 132 68.3) (size 0.8) (drill 0.4) (layers "F.Cu" "B.Cu") (free yes) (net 6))
 (via (at 152.8 92) (size 0.8) (drill 0.4) (layers "F.Cu" "B.Cu") (free yes) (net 6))
 (via (at 152.8 105.5) (size 0.8) (drill 0.4) (layers "F.Cu" "B.Cu") (free yes) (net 6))
 (via (at 118.5 111.7) (size 0.8) (drill 0.4) (layers "F.Cu" "B.Cu") (free yes) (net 6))
 (via (at 152.8 77) (size 0.8) (drill 0.4) (layers "F.Cu" "B.Cu") (free yes) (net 6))
 (via (at 124.5 111.7) (size 0.8) (drill 0.4) (layers "F.Cu" "B.Cu") (free yes) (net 6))
 (via (at 115.5 68.3) (size 0.8) (drill 0.4) (layers "F.Cu" "B.Cu") (free yes) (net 6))
 (via (at 123 68.3) (size 0.8) (drill 0.4) (layers "F.Cu" "B.Cu") (free yes) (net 6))
 (segment (start 138.725 97) (end 138.725 92.275) (width 1) (layer "F.Cu") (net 1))
 (segment (start 138.725 92.275) (end 139 92) (width 0.2) (layer "F.Cu") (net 1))
 (segment (start 139 92) (end 134.45 92) (width 1) (layer "F.Cu") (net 1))
 (segment (start 139 87) (end 139 92) (width 1) (layer "F.Cu") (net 1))
 (segment (start 134.45 92) (end 133.95 91.5) (width 0.2) (layer "F.Cu") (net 1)))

